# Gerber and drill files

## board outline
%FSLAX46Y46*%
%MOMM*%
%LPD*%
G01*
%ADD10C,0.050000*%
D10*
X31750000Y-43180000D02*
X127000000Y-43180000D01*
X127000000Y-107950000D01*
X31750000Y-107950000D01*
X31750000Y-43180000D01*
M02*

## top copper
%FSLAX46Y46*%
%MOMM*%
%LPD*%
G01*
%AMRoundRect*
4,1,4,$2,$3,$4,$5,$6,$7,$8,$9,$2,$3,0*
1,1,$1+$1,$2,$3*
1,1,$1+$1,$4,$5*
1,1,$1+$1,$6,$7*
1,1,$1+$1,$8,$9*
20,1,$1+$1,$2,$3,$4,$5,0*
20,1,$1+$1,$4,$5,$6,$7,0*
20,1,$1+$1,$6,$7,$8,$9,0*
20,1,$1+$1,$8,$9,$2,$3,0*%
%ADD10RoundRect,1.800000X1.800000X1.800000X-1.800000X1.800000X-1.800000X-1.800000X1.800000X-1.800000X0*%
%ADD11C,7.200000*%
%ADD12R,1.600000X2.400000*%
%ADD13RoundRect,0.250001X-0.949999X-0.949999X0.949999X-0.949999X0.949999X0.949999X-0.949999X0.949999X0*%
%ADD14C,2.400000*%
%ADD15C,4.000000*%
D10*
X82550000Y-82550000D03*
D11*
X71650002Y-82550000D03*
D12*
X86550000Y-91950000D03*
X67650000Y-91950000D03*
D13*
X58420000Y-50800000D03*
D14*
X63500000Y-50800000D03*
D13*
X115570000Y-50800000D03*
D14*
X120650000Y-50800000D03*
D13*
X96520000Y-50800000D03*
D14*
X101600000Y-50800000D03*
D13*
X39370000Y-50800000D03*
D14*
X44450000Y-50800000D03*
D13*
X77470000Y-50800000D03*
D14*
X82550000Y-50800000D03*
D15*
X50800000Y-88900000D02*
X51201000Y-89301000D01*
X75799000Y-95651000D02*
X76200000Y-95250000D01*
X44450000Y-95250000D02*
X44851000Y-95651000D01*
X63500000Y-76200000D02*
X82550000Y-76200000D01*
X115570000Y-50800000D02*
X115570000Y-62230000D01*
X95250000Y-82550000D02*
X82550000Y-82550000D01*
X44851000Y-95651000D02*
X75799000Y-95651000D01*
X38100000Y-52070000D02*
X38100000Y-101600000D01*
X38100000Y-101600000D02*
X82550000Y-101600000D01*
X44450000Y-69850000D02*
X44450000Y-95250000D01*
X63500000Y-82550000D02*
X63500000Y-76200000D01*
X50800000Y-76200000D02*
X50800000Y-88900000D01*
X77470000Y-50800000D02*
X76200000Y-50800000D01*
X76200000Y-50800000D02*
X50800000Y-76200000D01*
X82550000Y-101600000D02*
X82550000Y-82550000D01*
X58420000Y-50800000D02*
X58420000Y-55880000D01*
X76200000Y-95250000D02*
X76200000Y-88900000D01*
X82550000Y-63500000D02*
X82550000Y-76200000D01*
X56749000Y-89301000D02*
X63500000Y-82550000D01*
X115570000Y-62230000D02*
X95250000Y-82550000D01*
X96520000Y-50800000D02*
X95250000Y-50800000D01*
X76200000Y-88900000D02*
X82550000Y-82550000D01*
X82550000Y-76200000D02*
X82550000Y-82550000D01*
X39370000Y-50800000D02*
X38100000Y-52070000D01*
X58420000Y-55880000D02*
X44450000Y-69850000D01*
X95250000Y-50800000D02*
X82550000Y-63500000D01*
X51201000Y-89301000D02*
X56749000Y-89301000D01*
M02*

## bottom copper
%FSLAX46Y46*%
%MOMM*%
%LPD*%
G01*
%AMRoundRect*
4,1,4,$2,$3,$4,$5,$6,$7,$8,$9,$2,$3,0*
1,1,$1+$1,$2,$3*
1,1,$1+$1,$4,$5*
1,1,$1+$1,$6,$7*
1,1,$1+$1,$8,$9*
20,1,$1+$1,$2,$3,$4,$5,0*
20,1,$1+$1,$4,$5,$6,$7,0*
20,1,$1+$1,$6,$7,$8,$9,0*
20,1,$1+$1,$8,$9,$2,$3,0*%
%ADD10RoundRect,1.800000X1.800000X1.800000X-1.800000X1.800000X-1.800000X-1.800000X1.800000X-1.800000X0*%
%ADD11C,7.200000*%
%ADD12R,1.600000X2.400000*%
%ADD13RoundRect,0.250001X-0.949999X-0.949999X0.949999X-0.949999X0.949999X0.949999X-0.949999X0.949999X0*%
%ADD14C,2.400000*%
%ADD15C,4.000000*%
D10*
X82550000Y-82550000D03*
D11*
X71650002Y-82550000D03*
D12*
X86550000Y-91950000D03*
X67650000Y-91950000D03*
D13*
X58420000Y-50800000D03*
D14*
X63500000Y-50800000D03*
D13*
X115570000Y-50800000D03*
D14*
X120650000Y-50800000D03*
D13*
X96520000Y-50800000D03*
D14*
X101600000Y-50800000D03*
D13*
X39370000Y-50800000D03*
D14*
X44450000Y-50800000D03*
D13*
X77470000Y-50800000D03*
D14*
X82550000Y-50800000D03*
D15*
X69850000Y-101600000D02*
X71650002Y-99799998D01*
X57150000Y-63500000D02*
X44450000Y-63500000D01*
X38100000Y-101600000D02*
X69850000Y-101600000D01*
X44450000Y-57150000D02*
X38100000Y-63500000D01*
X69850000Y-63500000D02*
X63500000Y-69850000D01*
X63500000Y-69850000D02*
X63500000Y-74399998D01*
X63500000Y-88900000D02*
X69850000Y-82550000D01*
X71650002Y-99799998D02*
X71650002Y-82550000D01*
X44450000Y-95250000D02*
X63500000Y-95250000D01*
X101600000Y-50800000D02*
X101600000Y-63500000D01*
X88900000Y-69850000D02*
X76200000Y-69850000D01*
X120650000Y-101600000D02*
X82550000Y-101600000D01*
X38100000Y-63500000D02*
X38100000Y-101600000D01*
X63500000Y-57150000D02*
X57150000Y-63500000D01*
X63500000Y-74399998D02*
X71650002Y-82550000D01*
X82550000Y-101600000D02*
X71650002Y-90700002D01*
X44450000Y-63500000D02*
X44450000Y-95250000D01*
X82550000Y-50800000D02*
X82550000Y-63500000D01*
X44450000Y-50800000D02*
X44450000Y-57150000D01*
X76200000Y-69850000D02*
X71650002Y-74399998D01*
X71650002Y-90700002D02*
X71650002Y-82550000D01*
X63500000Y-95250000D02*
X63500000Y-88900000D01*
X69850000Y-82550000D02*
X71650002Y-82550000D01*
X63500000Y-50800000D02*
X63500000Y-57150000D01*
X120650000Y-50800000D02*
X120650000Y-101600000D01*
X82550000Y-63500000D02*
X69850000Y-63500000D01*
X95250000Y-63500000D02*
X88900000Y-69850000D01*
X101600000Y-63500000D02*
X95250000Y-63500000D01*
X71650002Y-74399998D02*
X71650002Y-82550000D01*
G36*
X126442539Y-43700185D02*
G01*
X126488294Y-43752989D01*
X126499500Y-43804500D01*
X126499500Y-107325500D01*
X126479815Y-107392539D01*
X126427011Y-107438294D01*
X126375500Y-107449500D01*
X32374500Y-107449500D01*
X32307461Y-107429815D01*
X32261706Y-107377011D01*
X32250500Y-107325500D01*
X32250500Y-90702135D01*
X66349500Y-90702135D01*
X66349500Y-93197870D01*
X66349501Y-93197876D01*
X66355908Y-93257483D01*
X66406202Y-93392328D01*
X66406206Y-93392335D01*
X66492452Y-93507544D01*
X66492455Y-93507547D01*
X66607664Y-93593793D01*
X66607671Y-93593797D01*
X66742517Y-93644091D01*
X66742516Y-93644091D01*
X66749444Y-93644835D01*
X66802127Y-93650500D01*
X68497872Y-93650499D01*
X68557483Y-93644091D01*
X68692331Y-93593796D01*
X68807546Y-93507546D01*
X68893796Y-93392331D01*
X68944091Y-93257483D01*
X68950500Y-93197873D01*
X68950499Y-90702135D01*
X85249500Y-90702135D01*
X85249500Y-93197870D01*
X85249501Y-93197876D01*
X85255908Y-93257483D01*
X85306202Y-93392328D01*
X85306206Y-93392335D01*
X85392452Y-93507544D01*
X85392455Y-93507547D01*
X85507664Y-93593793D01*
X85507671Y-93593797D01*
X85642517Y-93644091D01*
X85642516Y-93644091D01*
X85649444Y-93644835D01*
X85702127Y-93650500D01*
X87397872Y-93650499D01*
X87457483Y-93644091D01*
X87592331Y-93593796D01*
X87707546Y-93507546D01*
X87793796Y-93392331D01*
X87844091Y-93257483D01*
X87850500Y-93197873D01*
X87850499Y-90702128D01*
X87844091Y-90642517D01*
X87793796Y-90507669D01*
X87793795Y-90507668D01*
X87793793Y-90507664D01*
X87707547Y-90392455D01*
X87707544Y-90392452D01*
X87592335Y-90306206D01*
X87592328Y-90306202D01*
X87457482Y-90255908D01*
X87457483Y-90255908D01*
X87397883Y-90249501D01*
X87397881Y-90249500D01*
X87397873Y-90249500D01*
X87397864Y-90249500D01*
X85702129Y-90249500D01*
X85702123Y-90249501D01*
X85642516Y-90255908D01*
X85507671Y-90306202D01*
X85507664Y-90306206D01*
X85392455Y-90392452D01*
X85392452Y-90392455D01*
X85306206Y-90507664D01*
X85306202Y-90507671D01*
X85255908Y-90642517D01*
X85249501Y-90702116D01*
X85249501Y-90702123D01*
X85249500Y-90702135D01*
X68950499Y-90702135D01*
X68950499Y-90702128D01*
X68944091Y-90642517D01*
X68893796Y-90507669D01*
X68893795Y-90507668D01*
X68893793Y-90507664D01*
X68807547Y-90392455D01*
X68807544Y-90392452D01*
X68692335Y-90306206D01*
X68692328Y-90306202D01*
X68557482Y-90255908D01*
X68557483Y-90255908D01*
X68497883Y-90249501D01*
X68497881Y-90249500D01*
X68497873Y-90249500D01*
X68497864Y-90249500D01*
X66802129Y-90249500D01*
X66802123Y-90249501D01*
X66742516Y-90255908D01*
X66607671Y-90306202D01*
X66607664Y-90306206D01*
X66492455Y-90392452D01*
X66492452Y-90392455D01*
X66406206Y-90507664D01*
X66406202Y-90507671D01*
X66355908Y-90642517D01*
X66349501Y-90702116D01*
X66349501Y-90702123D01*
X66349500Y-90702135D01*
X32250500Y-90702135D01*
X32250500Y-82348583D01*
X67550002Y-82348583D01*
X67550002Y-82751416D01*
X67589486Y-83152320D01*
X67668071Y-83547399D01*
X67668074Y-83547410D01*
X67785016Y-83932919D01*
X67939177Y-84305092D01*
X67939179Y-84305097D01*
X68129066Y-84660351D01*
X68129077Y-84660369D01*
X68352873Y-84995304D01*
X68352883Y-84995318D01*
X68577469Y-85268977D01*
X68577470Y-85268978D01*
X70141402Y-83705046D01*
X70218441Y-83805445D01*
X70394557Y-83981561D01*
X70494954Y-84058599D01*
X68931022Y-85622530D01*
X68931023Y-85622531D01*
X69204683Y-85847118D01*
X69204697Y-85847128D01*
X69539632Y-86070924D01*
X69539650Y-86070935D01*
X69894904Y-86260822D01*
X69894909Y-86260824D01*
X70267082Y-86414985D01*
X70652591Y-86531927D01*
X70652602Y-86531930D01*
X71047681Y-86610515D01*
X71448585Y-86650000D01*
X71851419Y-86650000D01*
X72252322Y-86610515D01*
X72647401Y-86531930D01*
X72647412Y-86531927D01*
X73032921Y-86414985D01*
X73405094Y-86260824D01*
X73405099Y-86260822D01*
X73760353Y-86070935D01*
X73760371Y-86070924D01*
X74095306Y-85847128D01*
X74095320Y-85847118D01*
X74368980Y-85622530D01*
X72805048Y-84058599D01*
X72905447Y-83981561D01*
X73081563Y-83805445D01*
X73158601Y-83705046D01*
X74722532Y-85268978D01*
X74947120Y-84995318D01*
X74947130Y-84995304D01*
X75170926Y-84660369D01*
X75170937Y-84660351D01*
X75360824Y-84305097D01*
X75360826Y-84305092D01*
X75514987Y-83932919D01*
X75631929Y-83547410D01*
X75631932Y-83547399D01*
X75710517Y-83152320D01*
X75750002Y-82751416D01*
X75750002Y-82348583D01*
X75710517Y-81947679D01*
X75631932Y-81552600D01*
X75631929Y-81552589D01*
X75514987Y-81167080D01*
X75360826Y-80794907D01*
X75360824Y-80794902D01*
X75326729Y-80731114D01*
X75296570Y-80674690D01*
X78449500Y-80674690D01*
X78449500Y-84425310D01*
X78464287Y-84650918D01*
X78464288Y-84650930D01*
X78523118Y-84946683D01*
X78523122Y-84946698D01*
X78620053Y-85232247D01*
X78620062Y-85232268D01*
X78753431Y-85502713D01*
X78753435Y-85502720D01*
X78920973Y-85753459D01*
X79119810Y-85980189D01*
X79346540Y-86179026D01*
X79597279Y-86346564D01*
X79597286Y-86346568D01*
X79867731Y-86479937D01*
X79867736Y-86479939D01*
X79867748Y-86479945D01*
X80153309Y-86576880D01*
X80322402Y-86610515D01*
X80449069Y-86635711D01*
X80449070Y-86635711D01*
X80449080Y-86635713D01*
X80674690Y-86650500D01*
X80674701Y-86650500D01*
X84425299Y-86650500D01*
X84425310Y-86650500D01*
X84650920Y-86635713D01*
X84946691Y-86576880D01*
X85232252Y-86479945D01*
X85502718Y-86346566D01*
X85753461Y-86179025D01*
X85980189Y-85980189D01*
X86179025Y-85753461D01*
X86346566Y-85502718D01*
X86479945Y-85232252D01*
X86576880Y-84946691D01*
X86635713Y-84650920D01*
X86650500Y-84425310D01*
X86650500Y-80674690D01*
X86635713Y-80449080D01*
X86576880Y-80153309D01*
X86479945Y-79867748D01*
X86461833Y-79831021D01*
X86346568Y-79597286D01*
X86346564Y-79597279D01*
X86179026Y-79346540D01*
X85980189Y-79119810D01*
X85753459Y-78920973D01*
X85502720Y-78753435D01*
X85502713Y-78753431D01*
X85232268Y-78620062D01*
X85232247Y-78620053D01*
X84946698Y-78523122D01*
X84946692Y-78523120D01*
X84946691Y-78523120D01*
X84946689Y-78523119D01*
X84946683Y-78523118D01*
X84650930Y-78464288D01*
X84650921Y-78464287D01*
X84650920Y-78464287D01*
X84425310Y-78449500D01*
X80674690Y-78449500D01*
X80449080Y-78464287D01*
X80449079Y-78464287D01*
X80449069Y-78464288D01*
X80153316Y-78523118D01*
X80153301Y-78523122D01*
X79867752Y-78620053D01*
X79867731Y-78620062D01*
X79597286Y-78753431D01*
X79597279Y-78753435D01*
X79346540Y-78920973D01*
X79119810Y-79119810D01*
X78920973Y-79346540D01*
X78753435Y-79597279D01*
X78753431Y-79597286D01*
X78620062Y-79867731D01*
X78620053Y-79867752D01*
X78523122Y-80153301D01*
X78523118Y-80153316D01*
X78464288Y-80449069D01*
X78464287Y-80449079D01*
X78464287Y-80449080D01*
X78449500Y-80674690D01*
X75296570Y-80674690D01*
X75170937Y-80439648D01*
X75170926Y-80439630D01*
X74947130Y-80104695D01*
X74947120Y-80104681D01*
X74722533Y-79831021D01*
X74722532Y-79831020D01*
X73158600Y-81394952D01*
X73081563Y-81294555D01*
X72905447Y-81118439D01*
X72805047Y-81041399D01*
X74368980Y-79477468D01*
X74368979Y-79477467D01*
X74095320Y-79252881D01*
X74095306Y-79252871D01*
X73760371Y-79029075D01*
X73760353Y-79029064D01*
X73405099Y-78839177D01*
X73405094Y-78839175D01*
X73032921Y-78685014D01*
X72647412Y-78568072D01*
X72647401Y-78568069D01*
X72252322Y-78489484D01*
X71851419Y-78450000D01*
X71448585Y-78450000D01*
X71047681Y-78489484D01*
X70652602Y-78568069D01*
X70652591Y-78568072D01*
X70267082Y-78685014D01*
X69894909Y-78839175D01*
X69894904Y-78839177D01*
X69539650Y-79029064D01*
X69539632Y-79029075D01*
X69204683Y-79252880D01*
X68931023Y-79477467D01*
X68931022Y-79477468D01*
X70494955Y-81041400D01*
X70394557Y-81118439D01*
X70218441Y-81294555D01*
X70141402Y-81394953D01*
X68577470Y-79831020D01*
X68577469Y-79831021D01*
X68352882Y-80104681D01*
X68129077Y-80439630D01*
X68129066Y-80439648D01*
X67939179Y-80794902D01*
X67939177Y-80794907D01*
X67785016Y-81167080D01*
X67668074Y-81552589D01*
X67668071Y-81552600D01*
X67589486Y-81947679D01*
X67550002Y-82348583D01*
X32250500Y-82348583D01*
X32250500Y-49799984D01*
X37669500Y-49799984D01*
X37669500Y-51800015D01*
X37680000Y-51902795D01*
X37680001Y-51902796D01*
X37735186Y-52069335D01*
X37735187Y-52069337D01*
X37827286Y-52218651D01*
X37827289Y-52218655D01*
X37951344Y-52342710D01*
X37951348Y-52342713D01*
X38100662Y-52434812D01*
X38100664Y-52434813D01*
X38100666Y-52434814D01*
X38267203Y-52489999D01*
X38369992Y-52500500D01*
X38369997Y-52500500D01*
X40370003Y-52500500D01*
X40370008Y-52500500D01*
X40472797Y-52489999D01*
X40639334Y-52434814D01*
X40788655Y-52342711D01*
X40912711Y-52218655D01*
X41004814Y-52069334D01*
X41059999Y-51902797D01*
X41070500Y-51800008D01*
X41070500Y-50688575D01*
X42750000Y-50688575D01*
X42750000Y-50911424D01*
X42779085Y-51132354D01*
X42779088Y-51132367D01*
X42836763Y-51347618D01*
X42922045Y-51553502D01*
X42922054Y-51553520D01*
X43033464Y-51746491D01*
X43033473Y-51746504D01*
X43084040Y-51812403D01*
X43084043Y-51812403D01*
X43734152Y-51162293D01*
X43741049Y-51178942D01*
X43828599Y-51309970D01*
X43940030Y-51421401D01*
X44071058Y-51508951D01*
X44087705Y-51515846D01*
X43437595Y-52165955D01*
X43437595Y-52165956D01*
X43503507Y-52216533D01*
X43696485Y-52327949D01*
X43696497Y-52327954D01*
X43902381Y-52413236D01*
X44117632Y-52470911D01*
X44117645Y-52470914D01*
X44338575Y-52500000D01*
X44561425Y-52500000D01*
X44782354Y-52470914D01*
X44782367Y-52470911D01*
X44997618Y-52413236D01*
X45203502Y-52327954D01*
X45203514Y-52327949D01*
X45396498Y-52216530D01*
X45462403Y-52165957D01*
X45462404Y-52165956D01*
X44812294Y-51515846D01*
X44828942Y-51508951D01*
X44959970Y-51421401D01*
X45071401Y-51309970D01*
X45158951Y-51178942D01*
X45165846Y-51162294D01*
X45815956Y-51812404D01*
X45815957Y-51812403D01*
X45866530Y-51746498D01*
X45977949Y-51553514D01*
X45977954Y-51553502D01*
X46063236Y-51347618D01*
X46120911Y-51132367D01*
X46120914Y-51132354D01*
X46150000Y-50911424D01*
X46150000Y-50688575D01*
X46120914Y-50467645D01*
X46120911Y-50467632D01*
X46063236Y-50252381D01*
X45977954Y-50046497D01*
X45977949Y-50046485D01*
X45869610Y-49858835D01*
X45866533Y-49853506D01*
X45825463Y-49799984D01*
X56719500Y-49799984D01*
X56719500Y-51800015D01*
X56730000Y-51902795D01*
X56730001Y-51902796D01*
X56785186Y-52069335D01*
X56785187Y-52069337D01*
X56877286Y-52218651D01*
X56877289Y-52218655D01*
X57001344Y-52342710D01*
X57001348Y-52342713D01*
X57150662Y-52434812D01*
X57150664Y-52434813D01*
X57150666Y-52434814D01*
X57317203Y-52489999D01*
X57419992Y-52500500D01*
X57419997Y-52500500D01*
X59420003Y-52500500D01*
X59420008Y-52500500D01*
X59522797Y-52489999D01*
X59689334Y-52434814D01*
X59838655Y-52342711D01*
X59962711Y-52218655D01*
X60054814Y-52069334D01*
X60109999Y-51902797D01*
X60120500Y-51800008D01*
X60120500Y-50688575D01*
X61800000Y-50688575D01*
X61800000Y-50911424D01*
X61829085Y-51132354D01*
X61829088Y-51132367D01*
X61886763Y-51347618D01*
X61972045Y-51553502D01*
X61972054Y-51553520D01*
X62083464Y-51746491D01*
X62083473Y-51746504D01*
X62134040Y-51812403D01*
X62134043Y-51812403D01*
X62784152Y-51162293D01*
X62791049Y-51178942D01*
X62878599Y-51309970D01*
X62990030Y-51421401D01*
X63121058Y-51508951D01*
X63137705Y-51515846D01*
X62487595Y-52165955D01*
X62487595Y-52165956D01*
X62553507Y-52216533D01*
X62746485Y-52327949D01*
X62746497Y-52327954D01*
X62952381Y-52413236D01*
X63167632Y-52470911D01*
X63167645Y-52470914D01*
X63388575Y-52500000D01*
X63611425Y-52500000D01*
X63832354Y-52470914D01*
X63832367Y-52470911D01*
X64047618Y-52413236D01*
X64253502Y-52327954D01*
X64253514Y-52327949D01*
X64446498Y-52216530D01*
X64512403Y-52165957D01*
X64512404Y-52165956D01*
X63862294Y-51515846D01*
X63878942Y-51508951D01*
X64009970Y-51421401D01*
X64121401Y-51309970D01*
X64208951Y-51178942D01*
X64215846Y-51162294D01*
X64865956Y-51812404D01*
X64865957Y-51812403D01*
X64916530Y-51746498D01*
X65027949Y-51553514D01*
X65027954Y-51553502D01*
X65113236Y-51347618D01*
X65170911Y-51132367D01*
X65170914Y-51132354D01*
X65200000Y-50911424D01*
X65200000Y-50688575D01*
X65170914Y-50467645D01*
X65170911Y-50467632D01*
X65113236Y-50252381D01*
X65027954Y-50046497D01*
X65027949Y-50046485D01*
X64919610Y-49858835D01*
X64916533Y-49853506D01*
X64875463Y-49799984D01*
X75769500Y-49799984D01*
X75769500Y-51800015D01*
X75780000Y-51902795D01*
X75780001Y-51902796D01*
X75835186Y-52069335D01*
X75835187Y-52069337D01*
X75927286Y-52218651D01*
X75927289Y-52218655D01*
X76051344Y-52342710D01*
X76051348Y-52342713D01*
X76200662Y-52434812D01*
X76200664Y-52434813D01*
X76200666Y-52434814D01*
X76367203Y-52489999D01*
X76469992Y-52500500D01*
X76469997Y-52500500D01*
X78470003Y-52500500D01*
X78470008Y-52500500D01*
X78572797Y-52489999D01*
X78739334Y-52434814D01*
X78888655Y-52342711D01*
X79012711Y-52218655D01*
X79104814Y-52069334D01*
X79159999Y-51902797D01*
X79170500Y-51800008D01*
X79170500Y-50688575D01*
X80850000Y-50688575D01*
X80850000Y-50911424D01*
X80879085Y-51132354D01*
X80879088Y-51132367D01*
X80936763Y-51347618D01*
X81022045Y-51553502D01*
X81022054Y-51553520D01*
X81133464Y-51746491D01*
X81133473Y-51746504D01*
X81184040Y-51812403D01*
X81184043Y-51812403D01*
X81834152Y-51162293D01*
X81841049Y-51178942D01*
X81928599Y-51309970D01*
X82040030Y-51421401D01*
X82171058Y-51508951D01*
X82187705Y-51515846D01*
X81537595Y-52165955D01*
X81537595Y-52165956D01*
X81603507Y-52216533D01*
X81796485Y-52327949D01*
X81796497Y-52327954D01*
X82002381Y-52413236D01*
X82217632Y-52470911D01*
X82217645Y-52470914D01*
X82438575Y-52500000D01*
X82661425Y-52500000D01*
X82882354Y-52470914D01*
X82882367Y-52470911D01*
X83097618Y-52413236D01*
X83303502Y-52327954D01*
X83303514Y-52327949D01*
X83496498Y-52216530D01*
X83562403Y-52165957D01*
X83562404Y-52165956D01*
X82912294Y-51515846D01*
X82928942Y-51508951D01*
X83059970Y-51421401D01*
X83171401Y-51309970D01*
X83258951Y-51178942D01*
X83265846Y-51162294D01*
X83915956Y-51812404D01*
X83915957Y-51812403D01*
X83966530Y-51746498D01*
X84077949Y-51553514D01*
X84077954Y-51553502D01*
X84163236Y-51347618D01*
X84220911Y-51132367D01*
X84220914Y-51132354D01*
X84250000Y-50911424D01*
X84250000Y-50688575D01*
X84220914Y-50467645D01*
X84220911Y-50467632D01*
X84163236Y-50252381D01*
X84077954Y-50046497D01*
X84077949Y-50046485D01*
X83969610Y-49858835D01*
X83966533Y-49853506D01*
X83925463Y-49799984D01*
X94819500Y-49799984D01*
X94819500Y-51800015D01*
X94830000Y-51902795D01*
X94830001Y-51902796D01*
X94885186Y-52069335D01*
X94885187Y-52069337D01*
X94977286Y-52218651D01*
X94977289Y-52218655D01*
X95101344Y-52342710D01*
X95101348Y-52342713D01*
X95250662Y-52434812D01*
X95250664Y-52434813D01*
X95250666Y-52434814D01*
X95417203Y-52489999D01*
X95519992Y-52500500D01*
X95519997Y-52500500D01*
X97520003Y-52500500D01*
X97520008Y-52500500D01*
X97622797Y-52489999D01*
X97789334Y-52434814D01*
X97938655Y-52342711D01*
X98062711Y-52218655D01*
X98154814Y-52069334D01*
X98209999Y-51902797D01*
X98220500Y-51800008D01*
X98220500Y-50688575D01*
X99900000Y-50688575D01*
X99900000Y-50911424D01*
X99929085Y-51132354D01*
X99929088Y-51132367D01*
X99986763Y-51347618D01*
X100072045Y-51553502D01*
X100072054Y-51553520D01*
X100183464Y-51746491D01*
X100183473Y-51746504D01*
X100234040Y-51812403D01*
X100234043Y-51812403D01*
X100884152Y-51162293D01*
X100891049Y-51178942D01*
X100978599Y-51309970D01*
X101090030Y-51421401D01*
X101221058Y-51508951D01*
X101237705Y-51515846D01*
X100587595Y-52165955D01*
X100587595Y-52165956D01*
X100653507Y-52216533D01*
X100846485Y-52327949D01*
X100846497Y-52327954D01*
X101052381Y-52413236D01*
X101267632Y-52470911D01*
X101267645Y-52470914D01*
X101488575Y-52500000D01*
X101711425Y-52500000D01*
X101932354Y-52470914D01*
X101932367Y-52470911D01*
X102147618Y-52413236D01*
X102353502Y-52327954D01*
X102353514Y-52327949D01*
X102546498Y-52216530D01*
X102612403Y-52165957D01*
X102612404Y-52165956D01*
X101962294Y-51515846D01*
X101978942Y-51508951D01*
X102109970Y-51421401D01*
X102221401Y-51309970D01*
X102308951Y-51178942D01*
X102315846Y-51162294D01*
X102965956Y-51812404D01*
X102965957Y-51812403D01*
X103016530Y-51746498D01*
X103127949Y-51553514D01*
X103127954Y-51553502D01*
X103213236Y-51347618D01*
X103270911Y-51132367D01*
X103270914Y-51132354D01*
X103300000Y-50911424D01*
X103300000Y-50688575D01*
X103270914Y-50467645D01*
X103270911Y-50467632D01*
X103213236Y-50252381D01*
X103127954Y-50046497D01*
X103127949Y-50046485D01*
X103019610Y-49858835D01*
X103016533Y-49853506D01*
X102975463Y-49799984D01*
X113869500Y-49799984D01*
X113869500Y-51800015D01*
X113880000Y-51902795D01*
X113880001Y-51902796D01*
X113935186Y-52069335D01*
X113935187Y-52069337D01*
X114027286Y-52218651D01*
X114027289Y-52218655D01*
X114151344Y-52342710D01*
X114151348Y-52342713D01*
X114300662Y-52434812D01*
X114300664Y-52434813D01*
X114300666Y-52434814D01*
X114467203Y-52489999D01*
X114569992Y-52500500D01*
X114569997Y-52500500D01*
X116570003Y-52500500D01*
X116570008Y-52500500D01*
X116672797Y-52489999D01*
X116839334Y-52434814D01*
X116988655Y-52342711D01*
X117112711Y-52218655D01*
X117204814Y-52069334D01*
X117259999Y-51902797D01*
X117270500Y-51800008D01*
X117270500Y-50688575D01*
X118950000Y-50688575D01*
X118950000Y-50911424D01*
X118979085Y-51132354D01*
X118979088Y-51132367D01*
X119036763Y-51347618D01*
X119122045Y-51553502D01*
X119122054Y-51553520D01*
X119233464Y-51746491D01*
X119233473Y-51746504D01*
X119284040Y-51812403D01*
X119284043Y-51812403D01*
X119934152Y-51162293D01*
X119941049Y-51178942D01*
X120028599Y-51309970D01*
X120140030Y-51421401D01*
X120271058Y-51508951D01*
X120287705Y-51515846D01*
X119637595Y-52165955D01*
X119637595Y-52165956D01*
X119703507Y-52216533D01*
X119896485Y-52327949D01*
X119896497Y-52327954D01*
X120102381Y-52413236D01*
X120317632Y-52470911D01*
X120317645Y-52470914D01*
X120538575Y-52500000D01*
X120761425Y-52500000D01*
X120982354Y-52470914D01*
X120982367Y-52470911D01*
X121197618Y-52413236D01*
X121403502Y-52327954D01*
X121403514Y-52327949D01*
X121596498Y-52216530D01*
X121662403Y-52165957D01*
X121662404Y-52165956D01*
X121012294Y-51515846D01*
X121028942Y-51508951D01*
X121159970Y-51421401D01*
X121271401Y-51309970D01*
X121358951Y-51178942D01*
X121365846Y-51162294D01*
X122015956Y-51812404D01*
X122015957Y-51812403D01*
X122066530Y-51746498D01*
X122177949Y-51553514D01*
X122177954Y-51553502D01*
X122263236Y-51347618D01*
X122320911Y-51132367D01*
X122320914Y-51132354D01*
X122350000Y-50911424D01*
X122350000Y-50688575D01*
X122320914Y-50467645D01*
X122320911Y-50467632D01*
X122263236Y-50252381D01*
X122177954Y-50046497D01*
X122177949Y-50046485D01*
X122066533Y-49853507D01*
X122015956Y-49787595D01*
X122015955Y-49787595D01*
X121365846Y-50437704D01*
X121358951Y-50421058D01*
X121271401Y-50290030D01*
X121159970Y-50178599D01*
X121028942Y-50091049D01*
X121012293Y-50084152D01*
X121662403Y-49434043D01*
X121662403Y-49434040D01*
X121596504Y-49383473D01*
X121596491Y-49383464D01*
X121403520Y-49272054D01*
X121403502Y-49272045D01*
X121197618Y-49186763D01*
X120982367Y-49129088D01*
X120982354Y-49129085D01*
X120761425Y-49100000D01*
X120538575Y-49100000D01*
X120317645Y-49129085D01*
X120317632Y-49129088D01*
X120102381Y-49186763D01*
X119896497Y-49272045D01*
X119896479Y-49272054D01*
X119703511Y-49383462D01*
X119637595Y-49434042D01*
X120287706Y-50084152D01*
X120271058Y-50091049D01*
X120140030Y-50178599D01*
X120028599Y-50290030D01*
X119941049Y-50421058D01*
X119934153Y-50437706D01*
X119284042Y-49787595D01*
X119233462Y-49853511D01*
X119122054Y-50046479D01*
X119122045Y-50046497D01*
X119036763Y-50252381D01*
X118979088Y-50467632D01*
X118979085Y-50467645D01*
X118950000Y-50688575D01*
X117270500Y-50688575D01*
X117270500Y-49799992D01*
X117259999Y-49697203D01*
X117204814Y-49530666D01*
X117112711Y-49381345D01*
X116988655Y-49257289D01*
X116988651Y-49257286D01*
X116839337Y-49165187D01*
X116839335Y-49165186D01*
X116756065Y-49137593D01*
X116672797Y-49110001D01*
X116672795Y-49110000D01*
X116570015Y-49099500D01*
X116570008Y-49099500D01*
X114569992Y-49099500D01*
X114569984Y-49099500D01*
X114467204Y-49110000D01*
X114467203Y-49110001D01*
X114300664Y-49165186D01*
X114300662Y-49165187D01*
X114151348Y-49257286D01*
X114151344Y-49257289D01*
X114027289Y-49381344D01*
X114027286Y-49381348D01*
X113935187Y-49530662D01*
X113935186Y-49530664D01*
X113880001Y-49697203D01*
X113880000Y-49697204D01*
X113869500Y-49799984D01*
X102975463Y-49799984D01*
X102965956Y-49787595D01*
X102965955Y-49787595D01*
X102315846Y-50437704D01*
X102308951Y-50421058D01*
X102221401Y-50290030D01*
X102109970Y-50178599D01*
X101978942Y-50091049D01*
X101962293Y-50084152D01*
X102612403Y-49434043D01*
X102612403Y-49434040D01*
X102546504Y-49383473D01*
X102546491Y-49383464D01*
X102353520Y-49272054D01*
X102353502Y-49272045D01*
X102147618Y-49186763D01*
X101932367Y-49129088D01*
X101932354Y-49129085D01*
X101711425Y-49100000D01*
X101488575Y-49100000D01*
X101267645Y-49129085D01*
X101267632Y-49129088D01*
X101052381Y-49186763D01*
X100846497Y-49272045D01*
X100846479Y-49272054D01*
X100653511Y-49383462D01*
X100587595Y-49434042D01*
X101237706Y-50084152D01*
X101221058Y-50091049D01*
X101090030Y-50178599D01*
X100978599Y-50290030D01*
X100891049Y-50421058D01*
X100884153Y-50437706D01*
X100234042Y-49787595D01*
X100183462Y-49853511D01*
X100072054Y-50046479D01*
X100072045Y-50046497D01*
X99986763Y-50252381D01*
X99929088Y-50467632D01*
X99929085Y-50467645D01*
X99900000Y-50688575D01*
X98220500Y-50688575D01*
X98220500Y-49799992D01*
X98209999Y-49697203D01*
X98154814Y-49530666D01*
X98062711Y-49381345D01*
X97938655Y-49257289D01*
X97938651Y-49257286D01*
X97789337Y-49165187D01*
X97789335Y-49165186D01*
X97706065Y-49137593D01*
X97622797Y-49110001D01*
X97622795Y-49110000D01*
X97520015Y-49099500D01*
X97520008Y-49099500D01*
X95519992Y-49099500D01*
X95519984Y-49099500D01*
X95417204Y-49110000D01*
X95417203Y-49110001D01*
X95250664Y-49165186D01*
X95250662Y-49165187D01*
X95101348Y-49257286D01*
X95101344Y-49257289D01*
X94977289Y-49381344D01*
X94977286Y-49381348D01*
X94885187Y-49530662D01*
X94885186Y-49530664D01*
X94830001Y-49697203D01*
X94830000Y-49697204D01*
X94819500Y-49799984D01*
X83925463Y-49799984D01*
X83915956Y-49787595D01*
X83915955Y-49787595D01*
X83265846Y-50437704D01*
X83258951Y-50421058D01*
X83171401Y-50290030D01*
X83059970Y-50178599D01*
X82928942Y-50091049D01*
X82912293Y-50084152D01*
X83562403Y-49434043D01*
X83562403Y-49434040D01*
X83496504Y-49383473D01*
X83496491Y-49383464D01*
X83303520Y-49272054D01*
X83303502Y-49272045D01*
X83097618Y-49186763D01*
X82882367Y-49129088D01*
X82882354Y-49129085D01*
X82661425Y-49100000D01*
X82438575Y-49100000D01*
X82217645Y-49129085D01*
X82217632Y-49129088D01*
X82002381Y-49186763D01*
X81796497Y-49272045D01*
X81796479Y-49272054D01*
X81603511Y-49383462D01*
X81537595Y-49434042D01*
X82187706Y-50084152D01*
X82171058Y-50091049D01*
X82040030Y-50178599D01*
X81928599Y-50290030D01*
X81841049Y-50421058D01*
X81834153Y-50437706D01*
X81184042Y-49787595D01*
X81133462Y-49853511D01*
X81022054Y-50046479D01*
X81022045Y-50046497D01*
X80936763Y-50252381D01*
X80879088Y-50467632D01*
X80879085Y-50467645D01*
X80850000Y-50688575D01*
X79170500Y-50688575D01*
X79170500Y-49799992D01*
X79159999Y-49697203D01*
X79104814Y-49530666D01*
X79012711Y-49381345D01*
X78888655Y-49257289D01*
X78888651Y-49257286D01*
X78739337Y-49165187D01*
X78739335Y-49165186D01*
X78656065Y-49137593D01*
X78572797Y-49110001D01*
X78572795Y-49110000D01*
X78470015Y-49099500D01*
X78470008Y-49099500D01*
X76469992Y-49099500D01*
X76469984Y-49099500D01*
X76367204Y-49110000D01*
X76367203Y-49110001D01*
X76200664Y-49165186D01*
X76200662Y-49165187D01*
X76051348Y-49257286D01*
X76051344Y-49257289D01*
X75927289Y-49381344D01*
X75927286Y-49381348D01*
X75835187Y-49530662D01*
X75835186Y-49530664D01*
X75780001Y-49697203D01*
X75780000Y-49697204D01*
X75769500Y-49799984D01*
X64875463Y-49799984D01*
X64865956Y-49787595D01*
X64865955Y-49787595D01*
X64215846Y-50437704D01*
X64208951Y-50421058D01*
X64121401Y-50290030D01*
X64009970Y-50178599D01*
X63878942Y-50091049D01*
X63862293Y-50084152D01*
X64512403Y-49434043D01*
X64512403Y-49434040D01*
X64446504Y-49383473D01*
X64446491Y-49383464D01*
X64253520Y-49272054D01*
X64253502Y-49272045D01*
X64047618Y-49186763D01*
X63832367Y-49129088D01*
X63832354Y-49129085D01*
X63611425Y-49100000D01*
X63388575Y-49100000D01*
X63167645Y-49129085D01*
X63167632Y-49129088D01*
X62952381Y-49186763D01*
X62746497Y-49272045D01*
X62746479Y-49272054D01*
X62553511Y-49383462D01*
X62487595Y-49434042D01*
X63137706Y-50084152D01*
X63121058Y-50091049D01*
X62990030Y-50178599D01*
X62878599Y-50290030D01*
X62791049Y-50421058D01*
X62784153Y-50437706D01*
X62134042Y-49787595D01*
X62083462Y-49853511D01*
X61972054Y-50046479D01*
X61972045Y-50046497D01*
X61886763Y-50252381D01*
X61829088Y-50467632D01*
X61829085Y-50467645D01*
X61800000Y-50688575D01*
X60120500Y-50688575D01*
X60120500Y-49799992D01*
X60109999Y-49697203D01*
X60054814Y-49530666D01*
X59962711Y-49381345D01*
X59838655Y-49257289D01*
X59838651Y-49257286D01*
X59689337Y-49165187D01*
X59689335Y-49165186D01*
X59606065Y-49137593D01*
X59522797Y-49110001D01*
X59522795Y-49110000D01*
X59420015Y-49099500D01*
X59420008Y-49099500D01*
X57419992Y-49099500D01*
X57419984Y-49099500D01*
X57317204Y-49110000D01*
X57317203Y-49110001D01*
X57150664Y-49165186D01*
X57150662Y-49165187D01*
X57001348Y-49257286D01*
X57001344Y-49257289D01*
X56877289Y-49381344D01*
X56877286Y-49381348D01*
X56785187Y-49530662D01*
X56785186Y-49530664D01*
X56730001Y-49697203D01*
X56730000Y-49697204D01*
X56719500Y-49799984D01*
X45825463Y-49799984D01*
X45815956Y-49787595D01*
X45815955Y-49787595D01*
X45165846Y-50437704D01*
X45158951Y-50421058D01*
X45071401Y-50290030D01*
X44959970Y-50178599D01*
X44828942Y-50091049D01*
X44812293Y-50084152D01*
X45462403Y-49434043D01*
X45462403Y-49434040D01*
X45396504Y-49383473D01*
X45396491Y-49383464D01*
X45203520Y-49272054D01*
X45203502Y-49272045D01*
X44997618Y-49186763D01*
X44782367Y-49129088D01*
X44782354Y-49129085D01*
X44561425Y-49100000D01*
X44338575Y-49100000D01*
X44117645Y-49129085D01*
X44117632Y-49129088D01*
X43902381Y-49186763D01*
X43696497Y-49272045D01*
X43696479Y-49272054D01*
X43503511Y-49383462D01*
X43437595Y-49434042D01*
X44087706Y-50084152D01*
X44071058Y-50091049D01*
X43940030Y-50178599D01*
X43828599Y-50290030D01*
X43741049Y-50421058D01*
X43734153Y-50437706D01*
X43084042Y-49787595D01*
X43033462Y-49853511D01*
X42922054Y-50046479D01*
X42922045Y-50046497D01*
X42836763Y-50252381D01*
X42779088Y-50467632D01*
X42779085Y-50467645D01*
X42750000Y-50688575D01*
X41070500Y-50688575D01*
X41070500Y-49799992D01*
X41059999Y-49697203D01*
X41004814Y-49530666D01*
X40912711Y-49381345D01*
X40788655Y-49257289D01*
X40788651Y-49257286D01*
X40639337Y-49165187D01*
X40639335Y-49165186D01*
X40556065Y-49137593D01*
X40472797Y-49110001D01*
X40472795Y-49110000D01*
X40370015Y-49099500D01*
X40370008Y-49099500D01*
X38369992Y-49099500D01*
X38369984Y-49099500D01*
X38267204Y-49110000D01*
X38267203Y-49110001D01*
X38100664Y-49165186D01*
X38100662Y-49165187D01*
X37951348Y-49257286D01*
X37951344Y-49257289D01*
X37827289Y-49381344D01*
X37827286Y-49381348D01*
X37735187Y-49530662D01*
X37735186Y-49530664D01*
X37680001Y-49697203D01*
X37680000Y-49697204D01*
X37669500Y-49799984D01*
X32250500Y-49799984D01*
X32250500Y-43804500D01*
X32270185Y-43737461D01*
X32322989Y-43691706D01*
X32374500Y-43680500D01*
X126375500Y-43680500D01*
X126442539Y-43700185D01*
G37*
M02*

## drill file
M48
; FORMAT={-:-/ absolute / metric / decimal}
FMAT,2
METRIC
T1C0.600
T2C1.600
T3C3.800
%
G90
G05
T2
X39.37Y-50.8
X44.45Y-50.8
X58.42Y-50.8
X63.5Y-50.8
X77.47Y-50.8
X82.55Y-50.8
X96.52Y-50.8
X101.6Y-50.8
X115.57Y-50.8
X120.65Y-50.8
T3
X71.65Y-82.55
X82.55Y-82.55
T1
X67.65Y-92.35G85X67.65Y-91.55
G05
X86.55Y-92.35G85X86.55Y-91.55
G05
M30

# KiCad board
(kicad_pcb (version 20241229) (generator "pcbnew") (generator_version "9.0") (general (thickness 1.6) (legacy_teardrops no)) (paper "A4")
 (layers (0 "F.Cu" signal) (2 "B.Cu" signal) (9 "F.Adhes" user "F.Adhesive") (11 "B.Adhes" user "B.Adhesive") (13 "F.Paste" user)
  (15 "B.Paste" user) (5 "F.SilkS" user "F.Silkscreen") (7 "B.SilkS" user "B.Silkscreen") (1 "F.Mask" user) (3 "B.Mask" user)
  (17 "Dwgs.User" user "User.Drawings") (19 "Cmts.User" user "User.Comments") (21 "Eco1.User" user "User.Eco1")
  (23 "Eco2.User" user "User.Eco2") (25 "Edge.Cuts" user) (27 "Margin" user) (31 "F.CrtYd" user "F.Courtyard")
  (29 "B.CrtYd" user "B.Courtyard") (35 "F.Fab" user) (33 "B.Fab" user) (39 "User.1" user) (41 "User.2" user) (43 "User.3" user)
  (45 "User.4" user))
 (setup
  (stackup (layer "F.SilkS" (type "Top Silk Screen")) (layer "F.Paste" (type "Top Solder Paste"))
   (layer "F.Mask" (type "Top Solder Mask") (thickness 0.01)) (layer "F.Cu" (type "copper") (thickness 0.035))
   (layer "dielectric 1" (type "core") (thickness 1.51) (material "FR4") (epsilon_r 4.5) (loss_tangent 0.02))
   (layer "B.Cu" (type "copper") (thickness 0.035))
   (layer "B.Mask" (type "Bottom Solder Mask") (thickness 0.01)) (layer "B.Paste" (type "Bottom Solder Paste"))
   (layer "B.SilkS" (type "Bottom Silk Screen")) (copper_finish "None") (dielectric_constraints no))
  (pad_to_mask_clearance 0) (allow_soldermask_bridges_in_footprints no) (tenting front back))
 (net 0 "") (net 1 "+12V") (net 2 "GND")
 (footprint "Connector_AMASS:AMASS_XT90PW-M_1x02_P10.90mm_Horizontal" (layer "F.Cu") (at 82.55 82.55 180)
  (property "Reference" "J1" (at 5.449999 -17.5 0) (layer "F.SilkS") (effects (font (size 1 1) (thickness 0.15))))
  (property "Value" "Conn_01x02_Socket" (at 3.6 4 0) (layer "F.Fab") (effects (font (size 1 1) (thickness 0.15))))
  (pad "1" thru_hole roundrect (at 0 0 180) (size 7.2 7.2) (drill 3.8) (layers "*.Cu" "*.Mask") (remove_unused_layers no)
   (roundrect_rratio 0.25) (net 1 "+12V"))
  (pad "2" thru_hole circle (at 10.899998 0 180) (size 7.2 7.2) (drill 3.8) (layers "*.Cu" "*.Mask") (remove_unused_layers no) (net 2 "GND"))
  (pad "MP" thru_hole rect (at -4 -9.4 180) (size 1.6 2.4) (drill oval 0.6 1.4) (layers "*.Cu" "*.Mask") (remove_unused_layers no))
  (pad "MP" thru_hole rect (at 14.9 -9.4 180) (size 1.6 2.4) (drill oval 0.6 1.4) (layers "*.Cu" "*.Mask") (remove_unused_layers no)))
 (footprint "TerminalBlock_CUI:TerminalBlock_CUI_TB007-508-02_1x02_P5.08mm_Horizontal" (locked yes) (layer "F.Cu") (at 58.42 50.8)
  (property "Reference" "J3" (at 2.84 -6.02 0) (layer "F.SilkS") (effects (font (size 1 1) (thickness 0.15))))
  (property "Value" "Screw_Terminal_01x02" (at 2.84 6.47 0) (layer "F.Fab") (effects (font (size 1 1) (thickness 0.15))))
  (pad "1" thru_hole roundrect (at 0 0) (size 2.4 2.4) (drill 1.6) (layers "*.Cu" "*.Mask") (remove_unused_layers no)
   (roundrect_rratio 0.104167) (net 1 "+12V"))
  (pad "2" thru_hole circle (at 5.08 0) (size 2.4 2.4) (drill 1.6) (layers "*.Cu" "*.Mask") (remove_unused_layers no) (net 2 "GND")))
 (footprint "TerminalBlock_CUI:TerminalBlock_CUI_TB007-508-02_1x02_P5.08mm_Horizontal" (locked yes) (layer "F.Cu") (at 115.57 50.8)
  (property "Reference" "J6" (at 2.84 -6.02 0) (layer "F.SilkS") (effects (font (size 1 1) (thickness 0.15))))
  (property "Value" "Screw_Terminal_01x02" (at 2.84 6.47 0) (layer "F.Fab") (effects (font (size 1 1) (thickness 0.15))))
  (pad "1" thru_hole roundrect (at 0 0) (size 2.4 2.4) (drill 1.6) (layers "*.Cu" "*.Mask") (remove_unused_layers no)
   (roundrect_rratio 0.104167) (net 1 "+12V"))
  (pad "2" thru_hole circle (at 5.08 0) (size 2.4 2.4) (drill 1.6) (layers "*.Cu" "*.Mask") (remove_unused_layers no) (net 2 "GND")))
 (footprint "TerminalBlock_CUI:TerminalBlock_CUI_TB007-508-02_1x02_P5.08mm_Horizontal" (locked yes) (layer "F.Cu") (at 96.52 50.8)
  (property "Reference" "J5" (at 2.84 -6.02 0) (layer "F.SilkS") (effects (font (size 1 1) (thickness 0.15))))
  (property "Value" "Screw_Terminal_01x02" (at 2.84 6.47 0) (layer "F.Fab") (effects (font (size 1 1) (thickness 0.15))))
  (pad "1" thru_hole roundrect (at 0 0) (size 2.4 2.4) (drill 1.6) (layers "*.Cu" "*.Mask") (remove_unused_layers no)
   (roundrect_rratio 0.104167) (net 1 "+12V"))
  (pad "2" thru_hole circle (at 5.08 0) (size 2.4 2.4) (drill 1.6) (layers "*.Cu" "*.Mask") (remove_unused_layers no) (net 2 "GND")))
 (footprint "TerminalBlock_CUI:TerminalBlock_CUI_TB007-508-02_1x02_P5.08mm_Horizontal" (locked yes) (layer "F.Cu") (at 39.37 50.8)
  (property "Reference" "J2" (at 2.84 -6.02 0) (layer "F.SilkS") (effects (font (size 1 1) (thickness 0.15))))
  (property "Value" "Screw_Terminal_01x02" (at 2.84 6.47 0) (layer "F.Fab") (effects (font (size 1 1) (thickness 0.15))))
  (pad "1" thru_hole roundrect (at 0 0) (size 2.4 2.4) (drill 1.6) (layers "*.Cu" "*.Mask") (remove_unused_layers no)
   (roundrect_rratio 0.104167) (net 1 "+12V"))
  (pad "2" thru_hole circle (at 5.08 0) (size 2.4 2.4) (drill 1.6) (layers "*.Cu" "*.Mask") (remove_unused_layers no) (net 2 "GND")))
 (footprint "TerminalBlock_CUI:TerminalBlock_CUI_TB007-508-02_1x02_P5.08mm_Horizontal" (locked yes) (layer "F.Cu") (at 77.47 50.8)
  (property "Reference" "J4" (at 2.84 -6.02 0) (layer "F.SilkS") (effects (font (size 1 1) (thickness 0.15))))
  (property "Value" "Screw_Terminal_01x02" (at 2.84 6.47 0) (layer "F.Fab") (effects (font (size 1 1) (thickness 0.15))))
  (pad "1" thru_hole roundrect (at 0 0) (size 2.4 2.4) (drill 1.6) (layers "*.Cu" "*.Mask") (remove_unused_layers no)
   (roundrect_rratio 0.104167) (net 1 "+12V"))
  (pad "2" thru_hole circle (at 5.08 0) (size 2.4 2.4) (drill 1.6) (layers "*.Cu" "*.Mask") (remove_unused_layers no) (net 2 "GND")))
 (gr_rect (start 31.75 43.18) (end 127 107.95) (stroke (width 0.05) (type default)) (fill no) (layer "Edge.Cuts"))
 (segment (start 50.8 88.9) (end 51.201 89.301) (width 4) (layer "F.Cu") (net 1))
 (segment (start 75.799 95.651) (end 76.2 95.25) (width 4) (layer "F.Cu") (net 1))
 (segment (start 44.45 95.25) (end 44.851 95.651) (width 4) (layer "F.Cu") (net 1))
 (segment (start 63.5 76.2) (end 82.55 76.2) (width 4) (layer "F.Cu") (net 1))
 (segment (start 115.57 50.8) (end 115.57 62.23) (width 4) (layer "F.Cu") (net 1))
 (segment (start 95.25 82.55) (end 82.55 82.55) (width 4) (layer "F.Cu") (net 1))
 (segment (start 44.851 95.651) (end 75.799 95.651) (width 4) (layer "F.Cu") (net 1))
 (segment (start 38.1 52.07) (end 38.1 101.6) (width 4) (layer "F.Cu") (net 1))
 (segment (start 38.1 101.6) (end 82.55 101.6) (width 4) (layer "F.Cu") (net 1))
 (segment (start 44.45 69.85) (end 44.45 95.25) (width 4) (layer "F.Cu") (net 1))
 (segment (start 63.5 82.55) (end 63.5 76.2) (width 4) (layer "F.Cu") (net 1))
 (segment (start 50.8 76.2) (end 50.8 88.9) (width 4) (layer "F.Cu") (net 1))
 (segment (start 77.47 50.8) (end 76.2 50.8) (width 4) (layer "F.Cu") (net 1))
 (segment (start 76.2 50.8) (end 50.8 76.2) (width 4) (layer "F.Cu") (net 1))
 (segment (start 82.55 101.6) (end 82.55 82.55) (width 4) (layer "F.Cu") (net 1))
 (segment (start 58.42 50.8) (end 58.42 55.88) (width 4) (layer "F.Cu") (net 1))
 (segment (start 76.2 95.25) (end 76.2 88.9) (width 4) (layer "F.Cu") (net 1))
 (segment (start 82.55 63.5) (end 82.55 76.2) (width 4) (layer "F.Cu") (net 1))
 (segment (start 56.749 89.301) (end 63.5 82.55) (width 4) (layer "F.Cu") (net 1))
 (segment (start 115.57 62.23) (end 95.25 82.55) (width 4) (layer "F.Cu") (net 1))
 (segment (start 96.52 50.8) (end 95.25 50.8) (width 4) (layer "F.Cu") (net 1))
 (segment (start 76.2 88.9) (end 82.55 82.55) (width 4) (layer "F.Cu") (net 1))
 (segment (start 82.55 76.2) (end 82.55 82.55) (width 4) (layer "F.Cu") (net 1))
 (segment (start 39.37 50.8) (end 38.1 52.07) (width 4) (layer "F.Cu") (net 1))
 (segment (start 58.42 55.88) (end 44.45 69.85) (width 4) (layer "F.Cu") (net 1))
 (segment (start 95.25 50.8) (end 82.55 63.5) (width 4) (layer "F.Cu") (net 1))
 (segment (start 51.201 89.301) (end 56.749 89.301) (width 4) (layer "F.Cu") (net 1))
 (segment (start 69.85 101.6) (end 71.650002 99.799998) (width 4) (layer "B.Cu") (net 2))
 (segment (start 57.15 63.5) (end 44.45 63.5) (width 4) (layer "B.Cu") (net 2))
 (segment (start 38.1 101.6) (end 69.85 101.6) (width 4) (layer "B.Cu") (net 2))
 (segment (start 44.45 57.15) (end 38.1 63.5) (width 4) (layer "B.Cu") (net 2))
 (segment (start 69.85 63.5) (end 63.5 69.85) (width 4) (layer "B.Cu") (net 2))
 (segment (start 63.5 69.85) (end 63.5 74.399998) (width 4) (layer "B.Cu") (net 2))
 (segment (start 63.5 88.9) (end 69.85 82.55) (width 4) (layer "B.Cu") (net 2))
 (segment (start 71.650002 99.799998) (end 71.650002 82.55) (width 4) (layer "B.Cu") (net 2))
 (segment (start 44.45 95.25) (end 63.5 95.25) (width 4) (layer "B.Cu") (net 2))
 (segment (start 101.6 50.8) (end 101.6 63.5) (width 4) (layer "B.Cu") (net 2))
 (segment (start 88.9 69.85) (end 76.2 69.85) (width 4) (layer "B.Cu") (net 2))
 (segment (start 120.65 101.6) (end 82.55 101.6) (width 4) (layer "B.Cu") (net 2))
 (segment (start 38.1 63.5) (end 38.1 101.6) (width 4) (layer "B.Cu") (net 2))
 (segment (start 63.5 57.15) (end 57.15 63.5) (width 4) (layer "B.Cu") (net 2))
 (segment (start 63.5 74.399998) (end 71.650002 82.55) (width 4) (layer "B.Cu") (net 2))
 (segment (start 82.55 101.6) (end 71.650002 90.700002) (width 4) (layer "B.Cu") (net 2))
 (segment (start 44.45 63.5) (end 44.45 95.25) (width 4) (layer "B.Cu") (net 2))
 (segment (start 82.55 50.8) (end 82.55 63.5) (width 4) (layer "B.Cu") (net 2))
 (segment (start 44.45 50.8) (end 44.45 57.15) (width 4) (layer "B.Cu") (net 2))
 (segment (start 76.2 69.85) (end 71.650002 74.399998) (width 4) (layer "B.Cu") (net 2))
 (segment (start 71.650002 90.700002) (end 71.650002 82.55) (width 4) (layer "B.Cu") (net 2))
 (segment (start 63.5 95.25) (end 63.5 88.9) (width 4) (layer "B.Cu") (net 2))
 (segment (start 69.85 82.55) (end 71.650002 82.55) (width 4) (layer "B.Cu") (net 2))
 (segment (start 63.5 50.8) (end 63.5 57.15) (width 4) (layer "B.Cu") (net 2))
 (segment (start 120.65 50.8) (end 120.65 101.6) (width 4) (layer "B.Cu") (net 2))
 (segment (start 82.55 63.5) (end 69.85 63.5) (width 4) (layer "B.Cu") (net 2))
 (segment (start 95.25 63.5) (end 88.9 69.85) (width 4) (layer "B.Cu") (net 2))
 (segment (start 101.6 63.5) (end 95.25 63.5) (width 4) (layer "B.Cu") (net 2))
 (segment (start 71.650002 74.399998) (end 71.650002 82.55) (width 4) (layer "B.Cu") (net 2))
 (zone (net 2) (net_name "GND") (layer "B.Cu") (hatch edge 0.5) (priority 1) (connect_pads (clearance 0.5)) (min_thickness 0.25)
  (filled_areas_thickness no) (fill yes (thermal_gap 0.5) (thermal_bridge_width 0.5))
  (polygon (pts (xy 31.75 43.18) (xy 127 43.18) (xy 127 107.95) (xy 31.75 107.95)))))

